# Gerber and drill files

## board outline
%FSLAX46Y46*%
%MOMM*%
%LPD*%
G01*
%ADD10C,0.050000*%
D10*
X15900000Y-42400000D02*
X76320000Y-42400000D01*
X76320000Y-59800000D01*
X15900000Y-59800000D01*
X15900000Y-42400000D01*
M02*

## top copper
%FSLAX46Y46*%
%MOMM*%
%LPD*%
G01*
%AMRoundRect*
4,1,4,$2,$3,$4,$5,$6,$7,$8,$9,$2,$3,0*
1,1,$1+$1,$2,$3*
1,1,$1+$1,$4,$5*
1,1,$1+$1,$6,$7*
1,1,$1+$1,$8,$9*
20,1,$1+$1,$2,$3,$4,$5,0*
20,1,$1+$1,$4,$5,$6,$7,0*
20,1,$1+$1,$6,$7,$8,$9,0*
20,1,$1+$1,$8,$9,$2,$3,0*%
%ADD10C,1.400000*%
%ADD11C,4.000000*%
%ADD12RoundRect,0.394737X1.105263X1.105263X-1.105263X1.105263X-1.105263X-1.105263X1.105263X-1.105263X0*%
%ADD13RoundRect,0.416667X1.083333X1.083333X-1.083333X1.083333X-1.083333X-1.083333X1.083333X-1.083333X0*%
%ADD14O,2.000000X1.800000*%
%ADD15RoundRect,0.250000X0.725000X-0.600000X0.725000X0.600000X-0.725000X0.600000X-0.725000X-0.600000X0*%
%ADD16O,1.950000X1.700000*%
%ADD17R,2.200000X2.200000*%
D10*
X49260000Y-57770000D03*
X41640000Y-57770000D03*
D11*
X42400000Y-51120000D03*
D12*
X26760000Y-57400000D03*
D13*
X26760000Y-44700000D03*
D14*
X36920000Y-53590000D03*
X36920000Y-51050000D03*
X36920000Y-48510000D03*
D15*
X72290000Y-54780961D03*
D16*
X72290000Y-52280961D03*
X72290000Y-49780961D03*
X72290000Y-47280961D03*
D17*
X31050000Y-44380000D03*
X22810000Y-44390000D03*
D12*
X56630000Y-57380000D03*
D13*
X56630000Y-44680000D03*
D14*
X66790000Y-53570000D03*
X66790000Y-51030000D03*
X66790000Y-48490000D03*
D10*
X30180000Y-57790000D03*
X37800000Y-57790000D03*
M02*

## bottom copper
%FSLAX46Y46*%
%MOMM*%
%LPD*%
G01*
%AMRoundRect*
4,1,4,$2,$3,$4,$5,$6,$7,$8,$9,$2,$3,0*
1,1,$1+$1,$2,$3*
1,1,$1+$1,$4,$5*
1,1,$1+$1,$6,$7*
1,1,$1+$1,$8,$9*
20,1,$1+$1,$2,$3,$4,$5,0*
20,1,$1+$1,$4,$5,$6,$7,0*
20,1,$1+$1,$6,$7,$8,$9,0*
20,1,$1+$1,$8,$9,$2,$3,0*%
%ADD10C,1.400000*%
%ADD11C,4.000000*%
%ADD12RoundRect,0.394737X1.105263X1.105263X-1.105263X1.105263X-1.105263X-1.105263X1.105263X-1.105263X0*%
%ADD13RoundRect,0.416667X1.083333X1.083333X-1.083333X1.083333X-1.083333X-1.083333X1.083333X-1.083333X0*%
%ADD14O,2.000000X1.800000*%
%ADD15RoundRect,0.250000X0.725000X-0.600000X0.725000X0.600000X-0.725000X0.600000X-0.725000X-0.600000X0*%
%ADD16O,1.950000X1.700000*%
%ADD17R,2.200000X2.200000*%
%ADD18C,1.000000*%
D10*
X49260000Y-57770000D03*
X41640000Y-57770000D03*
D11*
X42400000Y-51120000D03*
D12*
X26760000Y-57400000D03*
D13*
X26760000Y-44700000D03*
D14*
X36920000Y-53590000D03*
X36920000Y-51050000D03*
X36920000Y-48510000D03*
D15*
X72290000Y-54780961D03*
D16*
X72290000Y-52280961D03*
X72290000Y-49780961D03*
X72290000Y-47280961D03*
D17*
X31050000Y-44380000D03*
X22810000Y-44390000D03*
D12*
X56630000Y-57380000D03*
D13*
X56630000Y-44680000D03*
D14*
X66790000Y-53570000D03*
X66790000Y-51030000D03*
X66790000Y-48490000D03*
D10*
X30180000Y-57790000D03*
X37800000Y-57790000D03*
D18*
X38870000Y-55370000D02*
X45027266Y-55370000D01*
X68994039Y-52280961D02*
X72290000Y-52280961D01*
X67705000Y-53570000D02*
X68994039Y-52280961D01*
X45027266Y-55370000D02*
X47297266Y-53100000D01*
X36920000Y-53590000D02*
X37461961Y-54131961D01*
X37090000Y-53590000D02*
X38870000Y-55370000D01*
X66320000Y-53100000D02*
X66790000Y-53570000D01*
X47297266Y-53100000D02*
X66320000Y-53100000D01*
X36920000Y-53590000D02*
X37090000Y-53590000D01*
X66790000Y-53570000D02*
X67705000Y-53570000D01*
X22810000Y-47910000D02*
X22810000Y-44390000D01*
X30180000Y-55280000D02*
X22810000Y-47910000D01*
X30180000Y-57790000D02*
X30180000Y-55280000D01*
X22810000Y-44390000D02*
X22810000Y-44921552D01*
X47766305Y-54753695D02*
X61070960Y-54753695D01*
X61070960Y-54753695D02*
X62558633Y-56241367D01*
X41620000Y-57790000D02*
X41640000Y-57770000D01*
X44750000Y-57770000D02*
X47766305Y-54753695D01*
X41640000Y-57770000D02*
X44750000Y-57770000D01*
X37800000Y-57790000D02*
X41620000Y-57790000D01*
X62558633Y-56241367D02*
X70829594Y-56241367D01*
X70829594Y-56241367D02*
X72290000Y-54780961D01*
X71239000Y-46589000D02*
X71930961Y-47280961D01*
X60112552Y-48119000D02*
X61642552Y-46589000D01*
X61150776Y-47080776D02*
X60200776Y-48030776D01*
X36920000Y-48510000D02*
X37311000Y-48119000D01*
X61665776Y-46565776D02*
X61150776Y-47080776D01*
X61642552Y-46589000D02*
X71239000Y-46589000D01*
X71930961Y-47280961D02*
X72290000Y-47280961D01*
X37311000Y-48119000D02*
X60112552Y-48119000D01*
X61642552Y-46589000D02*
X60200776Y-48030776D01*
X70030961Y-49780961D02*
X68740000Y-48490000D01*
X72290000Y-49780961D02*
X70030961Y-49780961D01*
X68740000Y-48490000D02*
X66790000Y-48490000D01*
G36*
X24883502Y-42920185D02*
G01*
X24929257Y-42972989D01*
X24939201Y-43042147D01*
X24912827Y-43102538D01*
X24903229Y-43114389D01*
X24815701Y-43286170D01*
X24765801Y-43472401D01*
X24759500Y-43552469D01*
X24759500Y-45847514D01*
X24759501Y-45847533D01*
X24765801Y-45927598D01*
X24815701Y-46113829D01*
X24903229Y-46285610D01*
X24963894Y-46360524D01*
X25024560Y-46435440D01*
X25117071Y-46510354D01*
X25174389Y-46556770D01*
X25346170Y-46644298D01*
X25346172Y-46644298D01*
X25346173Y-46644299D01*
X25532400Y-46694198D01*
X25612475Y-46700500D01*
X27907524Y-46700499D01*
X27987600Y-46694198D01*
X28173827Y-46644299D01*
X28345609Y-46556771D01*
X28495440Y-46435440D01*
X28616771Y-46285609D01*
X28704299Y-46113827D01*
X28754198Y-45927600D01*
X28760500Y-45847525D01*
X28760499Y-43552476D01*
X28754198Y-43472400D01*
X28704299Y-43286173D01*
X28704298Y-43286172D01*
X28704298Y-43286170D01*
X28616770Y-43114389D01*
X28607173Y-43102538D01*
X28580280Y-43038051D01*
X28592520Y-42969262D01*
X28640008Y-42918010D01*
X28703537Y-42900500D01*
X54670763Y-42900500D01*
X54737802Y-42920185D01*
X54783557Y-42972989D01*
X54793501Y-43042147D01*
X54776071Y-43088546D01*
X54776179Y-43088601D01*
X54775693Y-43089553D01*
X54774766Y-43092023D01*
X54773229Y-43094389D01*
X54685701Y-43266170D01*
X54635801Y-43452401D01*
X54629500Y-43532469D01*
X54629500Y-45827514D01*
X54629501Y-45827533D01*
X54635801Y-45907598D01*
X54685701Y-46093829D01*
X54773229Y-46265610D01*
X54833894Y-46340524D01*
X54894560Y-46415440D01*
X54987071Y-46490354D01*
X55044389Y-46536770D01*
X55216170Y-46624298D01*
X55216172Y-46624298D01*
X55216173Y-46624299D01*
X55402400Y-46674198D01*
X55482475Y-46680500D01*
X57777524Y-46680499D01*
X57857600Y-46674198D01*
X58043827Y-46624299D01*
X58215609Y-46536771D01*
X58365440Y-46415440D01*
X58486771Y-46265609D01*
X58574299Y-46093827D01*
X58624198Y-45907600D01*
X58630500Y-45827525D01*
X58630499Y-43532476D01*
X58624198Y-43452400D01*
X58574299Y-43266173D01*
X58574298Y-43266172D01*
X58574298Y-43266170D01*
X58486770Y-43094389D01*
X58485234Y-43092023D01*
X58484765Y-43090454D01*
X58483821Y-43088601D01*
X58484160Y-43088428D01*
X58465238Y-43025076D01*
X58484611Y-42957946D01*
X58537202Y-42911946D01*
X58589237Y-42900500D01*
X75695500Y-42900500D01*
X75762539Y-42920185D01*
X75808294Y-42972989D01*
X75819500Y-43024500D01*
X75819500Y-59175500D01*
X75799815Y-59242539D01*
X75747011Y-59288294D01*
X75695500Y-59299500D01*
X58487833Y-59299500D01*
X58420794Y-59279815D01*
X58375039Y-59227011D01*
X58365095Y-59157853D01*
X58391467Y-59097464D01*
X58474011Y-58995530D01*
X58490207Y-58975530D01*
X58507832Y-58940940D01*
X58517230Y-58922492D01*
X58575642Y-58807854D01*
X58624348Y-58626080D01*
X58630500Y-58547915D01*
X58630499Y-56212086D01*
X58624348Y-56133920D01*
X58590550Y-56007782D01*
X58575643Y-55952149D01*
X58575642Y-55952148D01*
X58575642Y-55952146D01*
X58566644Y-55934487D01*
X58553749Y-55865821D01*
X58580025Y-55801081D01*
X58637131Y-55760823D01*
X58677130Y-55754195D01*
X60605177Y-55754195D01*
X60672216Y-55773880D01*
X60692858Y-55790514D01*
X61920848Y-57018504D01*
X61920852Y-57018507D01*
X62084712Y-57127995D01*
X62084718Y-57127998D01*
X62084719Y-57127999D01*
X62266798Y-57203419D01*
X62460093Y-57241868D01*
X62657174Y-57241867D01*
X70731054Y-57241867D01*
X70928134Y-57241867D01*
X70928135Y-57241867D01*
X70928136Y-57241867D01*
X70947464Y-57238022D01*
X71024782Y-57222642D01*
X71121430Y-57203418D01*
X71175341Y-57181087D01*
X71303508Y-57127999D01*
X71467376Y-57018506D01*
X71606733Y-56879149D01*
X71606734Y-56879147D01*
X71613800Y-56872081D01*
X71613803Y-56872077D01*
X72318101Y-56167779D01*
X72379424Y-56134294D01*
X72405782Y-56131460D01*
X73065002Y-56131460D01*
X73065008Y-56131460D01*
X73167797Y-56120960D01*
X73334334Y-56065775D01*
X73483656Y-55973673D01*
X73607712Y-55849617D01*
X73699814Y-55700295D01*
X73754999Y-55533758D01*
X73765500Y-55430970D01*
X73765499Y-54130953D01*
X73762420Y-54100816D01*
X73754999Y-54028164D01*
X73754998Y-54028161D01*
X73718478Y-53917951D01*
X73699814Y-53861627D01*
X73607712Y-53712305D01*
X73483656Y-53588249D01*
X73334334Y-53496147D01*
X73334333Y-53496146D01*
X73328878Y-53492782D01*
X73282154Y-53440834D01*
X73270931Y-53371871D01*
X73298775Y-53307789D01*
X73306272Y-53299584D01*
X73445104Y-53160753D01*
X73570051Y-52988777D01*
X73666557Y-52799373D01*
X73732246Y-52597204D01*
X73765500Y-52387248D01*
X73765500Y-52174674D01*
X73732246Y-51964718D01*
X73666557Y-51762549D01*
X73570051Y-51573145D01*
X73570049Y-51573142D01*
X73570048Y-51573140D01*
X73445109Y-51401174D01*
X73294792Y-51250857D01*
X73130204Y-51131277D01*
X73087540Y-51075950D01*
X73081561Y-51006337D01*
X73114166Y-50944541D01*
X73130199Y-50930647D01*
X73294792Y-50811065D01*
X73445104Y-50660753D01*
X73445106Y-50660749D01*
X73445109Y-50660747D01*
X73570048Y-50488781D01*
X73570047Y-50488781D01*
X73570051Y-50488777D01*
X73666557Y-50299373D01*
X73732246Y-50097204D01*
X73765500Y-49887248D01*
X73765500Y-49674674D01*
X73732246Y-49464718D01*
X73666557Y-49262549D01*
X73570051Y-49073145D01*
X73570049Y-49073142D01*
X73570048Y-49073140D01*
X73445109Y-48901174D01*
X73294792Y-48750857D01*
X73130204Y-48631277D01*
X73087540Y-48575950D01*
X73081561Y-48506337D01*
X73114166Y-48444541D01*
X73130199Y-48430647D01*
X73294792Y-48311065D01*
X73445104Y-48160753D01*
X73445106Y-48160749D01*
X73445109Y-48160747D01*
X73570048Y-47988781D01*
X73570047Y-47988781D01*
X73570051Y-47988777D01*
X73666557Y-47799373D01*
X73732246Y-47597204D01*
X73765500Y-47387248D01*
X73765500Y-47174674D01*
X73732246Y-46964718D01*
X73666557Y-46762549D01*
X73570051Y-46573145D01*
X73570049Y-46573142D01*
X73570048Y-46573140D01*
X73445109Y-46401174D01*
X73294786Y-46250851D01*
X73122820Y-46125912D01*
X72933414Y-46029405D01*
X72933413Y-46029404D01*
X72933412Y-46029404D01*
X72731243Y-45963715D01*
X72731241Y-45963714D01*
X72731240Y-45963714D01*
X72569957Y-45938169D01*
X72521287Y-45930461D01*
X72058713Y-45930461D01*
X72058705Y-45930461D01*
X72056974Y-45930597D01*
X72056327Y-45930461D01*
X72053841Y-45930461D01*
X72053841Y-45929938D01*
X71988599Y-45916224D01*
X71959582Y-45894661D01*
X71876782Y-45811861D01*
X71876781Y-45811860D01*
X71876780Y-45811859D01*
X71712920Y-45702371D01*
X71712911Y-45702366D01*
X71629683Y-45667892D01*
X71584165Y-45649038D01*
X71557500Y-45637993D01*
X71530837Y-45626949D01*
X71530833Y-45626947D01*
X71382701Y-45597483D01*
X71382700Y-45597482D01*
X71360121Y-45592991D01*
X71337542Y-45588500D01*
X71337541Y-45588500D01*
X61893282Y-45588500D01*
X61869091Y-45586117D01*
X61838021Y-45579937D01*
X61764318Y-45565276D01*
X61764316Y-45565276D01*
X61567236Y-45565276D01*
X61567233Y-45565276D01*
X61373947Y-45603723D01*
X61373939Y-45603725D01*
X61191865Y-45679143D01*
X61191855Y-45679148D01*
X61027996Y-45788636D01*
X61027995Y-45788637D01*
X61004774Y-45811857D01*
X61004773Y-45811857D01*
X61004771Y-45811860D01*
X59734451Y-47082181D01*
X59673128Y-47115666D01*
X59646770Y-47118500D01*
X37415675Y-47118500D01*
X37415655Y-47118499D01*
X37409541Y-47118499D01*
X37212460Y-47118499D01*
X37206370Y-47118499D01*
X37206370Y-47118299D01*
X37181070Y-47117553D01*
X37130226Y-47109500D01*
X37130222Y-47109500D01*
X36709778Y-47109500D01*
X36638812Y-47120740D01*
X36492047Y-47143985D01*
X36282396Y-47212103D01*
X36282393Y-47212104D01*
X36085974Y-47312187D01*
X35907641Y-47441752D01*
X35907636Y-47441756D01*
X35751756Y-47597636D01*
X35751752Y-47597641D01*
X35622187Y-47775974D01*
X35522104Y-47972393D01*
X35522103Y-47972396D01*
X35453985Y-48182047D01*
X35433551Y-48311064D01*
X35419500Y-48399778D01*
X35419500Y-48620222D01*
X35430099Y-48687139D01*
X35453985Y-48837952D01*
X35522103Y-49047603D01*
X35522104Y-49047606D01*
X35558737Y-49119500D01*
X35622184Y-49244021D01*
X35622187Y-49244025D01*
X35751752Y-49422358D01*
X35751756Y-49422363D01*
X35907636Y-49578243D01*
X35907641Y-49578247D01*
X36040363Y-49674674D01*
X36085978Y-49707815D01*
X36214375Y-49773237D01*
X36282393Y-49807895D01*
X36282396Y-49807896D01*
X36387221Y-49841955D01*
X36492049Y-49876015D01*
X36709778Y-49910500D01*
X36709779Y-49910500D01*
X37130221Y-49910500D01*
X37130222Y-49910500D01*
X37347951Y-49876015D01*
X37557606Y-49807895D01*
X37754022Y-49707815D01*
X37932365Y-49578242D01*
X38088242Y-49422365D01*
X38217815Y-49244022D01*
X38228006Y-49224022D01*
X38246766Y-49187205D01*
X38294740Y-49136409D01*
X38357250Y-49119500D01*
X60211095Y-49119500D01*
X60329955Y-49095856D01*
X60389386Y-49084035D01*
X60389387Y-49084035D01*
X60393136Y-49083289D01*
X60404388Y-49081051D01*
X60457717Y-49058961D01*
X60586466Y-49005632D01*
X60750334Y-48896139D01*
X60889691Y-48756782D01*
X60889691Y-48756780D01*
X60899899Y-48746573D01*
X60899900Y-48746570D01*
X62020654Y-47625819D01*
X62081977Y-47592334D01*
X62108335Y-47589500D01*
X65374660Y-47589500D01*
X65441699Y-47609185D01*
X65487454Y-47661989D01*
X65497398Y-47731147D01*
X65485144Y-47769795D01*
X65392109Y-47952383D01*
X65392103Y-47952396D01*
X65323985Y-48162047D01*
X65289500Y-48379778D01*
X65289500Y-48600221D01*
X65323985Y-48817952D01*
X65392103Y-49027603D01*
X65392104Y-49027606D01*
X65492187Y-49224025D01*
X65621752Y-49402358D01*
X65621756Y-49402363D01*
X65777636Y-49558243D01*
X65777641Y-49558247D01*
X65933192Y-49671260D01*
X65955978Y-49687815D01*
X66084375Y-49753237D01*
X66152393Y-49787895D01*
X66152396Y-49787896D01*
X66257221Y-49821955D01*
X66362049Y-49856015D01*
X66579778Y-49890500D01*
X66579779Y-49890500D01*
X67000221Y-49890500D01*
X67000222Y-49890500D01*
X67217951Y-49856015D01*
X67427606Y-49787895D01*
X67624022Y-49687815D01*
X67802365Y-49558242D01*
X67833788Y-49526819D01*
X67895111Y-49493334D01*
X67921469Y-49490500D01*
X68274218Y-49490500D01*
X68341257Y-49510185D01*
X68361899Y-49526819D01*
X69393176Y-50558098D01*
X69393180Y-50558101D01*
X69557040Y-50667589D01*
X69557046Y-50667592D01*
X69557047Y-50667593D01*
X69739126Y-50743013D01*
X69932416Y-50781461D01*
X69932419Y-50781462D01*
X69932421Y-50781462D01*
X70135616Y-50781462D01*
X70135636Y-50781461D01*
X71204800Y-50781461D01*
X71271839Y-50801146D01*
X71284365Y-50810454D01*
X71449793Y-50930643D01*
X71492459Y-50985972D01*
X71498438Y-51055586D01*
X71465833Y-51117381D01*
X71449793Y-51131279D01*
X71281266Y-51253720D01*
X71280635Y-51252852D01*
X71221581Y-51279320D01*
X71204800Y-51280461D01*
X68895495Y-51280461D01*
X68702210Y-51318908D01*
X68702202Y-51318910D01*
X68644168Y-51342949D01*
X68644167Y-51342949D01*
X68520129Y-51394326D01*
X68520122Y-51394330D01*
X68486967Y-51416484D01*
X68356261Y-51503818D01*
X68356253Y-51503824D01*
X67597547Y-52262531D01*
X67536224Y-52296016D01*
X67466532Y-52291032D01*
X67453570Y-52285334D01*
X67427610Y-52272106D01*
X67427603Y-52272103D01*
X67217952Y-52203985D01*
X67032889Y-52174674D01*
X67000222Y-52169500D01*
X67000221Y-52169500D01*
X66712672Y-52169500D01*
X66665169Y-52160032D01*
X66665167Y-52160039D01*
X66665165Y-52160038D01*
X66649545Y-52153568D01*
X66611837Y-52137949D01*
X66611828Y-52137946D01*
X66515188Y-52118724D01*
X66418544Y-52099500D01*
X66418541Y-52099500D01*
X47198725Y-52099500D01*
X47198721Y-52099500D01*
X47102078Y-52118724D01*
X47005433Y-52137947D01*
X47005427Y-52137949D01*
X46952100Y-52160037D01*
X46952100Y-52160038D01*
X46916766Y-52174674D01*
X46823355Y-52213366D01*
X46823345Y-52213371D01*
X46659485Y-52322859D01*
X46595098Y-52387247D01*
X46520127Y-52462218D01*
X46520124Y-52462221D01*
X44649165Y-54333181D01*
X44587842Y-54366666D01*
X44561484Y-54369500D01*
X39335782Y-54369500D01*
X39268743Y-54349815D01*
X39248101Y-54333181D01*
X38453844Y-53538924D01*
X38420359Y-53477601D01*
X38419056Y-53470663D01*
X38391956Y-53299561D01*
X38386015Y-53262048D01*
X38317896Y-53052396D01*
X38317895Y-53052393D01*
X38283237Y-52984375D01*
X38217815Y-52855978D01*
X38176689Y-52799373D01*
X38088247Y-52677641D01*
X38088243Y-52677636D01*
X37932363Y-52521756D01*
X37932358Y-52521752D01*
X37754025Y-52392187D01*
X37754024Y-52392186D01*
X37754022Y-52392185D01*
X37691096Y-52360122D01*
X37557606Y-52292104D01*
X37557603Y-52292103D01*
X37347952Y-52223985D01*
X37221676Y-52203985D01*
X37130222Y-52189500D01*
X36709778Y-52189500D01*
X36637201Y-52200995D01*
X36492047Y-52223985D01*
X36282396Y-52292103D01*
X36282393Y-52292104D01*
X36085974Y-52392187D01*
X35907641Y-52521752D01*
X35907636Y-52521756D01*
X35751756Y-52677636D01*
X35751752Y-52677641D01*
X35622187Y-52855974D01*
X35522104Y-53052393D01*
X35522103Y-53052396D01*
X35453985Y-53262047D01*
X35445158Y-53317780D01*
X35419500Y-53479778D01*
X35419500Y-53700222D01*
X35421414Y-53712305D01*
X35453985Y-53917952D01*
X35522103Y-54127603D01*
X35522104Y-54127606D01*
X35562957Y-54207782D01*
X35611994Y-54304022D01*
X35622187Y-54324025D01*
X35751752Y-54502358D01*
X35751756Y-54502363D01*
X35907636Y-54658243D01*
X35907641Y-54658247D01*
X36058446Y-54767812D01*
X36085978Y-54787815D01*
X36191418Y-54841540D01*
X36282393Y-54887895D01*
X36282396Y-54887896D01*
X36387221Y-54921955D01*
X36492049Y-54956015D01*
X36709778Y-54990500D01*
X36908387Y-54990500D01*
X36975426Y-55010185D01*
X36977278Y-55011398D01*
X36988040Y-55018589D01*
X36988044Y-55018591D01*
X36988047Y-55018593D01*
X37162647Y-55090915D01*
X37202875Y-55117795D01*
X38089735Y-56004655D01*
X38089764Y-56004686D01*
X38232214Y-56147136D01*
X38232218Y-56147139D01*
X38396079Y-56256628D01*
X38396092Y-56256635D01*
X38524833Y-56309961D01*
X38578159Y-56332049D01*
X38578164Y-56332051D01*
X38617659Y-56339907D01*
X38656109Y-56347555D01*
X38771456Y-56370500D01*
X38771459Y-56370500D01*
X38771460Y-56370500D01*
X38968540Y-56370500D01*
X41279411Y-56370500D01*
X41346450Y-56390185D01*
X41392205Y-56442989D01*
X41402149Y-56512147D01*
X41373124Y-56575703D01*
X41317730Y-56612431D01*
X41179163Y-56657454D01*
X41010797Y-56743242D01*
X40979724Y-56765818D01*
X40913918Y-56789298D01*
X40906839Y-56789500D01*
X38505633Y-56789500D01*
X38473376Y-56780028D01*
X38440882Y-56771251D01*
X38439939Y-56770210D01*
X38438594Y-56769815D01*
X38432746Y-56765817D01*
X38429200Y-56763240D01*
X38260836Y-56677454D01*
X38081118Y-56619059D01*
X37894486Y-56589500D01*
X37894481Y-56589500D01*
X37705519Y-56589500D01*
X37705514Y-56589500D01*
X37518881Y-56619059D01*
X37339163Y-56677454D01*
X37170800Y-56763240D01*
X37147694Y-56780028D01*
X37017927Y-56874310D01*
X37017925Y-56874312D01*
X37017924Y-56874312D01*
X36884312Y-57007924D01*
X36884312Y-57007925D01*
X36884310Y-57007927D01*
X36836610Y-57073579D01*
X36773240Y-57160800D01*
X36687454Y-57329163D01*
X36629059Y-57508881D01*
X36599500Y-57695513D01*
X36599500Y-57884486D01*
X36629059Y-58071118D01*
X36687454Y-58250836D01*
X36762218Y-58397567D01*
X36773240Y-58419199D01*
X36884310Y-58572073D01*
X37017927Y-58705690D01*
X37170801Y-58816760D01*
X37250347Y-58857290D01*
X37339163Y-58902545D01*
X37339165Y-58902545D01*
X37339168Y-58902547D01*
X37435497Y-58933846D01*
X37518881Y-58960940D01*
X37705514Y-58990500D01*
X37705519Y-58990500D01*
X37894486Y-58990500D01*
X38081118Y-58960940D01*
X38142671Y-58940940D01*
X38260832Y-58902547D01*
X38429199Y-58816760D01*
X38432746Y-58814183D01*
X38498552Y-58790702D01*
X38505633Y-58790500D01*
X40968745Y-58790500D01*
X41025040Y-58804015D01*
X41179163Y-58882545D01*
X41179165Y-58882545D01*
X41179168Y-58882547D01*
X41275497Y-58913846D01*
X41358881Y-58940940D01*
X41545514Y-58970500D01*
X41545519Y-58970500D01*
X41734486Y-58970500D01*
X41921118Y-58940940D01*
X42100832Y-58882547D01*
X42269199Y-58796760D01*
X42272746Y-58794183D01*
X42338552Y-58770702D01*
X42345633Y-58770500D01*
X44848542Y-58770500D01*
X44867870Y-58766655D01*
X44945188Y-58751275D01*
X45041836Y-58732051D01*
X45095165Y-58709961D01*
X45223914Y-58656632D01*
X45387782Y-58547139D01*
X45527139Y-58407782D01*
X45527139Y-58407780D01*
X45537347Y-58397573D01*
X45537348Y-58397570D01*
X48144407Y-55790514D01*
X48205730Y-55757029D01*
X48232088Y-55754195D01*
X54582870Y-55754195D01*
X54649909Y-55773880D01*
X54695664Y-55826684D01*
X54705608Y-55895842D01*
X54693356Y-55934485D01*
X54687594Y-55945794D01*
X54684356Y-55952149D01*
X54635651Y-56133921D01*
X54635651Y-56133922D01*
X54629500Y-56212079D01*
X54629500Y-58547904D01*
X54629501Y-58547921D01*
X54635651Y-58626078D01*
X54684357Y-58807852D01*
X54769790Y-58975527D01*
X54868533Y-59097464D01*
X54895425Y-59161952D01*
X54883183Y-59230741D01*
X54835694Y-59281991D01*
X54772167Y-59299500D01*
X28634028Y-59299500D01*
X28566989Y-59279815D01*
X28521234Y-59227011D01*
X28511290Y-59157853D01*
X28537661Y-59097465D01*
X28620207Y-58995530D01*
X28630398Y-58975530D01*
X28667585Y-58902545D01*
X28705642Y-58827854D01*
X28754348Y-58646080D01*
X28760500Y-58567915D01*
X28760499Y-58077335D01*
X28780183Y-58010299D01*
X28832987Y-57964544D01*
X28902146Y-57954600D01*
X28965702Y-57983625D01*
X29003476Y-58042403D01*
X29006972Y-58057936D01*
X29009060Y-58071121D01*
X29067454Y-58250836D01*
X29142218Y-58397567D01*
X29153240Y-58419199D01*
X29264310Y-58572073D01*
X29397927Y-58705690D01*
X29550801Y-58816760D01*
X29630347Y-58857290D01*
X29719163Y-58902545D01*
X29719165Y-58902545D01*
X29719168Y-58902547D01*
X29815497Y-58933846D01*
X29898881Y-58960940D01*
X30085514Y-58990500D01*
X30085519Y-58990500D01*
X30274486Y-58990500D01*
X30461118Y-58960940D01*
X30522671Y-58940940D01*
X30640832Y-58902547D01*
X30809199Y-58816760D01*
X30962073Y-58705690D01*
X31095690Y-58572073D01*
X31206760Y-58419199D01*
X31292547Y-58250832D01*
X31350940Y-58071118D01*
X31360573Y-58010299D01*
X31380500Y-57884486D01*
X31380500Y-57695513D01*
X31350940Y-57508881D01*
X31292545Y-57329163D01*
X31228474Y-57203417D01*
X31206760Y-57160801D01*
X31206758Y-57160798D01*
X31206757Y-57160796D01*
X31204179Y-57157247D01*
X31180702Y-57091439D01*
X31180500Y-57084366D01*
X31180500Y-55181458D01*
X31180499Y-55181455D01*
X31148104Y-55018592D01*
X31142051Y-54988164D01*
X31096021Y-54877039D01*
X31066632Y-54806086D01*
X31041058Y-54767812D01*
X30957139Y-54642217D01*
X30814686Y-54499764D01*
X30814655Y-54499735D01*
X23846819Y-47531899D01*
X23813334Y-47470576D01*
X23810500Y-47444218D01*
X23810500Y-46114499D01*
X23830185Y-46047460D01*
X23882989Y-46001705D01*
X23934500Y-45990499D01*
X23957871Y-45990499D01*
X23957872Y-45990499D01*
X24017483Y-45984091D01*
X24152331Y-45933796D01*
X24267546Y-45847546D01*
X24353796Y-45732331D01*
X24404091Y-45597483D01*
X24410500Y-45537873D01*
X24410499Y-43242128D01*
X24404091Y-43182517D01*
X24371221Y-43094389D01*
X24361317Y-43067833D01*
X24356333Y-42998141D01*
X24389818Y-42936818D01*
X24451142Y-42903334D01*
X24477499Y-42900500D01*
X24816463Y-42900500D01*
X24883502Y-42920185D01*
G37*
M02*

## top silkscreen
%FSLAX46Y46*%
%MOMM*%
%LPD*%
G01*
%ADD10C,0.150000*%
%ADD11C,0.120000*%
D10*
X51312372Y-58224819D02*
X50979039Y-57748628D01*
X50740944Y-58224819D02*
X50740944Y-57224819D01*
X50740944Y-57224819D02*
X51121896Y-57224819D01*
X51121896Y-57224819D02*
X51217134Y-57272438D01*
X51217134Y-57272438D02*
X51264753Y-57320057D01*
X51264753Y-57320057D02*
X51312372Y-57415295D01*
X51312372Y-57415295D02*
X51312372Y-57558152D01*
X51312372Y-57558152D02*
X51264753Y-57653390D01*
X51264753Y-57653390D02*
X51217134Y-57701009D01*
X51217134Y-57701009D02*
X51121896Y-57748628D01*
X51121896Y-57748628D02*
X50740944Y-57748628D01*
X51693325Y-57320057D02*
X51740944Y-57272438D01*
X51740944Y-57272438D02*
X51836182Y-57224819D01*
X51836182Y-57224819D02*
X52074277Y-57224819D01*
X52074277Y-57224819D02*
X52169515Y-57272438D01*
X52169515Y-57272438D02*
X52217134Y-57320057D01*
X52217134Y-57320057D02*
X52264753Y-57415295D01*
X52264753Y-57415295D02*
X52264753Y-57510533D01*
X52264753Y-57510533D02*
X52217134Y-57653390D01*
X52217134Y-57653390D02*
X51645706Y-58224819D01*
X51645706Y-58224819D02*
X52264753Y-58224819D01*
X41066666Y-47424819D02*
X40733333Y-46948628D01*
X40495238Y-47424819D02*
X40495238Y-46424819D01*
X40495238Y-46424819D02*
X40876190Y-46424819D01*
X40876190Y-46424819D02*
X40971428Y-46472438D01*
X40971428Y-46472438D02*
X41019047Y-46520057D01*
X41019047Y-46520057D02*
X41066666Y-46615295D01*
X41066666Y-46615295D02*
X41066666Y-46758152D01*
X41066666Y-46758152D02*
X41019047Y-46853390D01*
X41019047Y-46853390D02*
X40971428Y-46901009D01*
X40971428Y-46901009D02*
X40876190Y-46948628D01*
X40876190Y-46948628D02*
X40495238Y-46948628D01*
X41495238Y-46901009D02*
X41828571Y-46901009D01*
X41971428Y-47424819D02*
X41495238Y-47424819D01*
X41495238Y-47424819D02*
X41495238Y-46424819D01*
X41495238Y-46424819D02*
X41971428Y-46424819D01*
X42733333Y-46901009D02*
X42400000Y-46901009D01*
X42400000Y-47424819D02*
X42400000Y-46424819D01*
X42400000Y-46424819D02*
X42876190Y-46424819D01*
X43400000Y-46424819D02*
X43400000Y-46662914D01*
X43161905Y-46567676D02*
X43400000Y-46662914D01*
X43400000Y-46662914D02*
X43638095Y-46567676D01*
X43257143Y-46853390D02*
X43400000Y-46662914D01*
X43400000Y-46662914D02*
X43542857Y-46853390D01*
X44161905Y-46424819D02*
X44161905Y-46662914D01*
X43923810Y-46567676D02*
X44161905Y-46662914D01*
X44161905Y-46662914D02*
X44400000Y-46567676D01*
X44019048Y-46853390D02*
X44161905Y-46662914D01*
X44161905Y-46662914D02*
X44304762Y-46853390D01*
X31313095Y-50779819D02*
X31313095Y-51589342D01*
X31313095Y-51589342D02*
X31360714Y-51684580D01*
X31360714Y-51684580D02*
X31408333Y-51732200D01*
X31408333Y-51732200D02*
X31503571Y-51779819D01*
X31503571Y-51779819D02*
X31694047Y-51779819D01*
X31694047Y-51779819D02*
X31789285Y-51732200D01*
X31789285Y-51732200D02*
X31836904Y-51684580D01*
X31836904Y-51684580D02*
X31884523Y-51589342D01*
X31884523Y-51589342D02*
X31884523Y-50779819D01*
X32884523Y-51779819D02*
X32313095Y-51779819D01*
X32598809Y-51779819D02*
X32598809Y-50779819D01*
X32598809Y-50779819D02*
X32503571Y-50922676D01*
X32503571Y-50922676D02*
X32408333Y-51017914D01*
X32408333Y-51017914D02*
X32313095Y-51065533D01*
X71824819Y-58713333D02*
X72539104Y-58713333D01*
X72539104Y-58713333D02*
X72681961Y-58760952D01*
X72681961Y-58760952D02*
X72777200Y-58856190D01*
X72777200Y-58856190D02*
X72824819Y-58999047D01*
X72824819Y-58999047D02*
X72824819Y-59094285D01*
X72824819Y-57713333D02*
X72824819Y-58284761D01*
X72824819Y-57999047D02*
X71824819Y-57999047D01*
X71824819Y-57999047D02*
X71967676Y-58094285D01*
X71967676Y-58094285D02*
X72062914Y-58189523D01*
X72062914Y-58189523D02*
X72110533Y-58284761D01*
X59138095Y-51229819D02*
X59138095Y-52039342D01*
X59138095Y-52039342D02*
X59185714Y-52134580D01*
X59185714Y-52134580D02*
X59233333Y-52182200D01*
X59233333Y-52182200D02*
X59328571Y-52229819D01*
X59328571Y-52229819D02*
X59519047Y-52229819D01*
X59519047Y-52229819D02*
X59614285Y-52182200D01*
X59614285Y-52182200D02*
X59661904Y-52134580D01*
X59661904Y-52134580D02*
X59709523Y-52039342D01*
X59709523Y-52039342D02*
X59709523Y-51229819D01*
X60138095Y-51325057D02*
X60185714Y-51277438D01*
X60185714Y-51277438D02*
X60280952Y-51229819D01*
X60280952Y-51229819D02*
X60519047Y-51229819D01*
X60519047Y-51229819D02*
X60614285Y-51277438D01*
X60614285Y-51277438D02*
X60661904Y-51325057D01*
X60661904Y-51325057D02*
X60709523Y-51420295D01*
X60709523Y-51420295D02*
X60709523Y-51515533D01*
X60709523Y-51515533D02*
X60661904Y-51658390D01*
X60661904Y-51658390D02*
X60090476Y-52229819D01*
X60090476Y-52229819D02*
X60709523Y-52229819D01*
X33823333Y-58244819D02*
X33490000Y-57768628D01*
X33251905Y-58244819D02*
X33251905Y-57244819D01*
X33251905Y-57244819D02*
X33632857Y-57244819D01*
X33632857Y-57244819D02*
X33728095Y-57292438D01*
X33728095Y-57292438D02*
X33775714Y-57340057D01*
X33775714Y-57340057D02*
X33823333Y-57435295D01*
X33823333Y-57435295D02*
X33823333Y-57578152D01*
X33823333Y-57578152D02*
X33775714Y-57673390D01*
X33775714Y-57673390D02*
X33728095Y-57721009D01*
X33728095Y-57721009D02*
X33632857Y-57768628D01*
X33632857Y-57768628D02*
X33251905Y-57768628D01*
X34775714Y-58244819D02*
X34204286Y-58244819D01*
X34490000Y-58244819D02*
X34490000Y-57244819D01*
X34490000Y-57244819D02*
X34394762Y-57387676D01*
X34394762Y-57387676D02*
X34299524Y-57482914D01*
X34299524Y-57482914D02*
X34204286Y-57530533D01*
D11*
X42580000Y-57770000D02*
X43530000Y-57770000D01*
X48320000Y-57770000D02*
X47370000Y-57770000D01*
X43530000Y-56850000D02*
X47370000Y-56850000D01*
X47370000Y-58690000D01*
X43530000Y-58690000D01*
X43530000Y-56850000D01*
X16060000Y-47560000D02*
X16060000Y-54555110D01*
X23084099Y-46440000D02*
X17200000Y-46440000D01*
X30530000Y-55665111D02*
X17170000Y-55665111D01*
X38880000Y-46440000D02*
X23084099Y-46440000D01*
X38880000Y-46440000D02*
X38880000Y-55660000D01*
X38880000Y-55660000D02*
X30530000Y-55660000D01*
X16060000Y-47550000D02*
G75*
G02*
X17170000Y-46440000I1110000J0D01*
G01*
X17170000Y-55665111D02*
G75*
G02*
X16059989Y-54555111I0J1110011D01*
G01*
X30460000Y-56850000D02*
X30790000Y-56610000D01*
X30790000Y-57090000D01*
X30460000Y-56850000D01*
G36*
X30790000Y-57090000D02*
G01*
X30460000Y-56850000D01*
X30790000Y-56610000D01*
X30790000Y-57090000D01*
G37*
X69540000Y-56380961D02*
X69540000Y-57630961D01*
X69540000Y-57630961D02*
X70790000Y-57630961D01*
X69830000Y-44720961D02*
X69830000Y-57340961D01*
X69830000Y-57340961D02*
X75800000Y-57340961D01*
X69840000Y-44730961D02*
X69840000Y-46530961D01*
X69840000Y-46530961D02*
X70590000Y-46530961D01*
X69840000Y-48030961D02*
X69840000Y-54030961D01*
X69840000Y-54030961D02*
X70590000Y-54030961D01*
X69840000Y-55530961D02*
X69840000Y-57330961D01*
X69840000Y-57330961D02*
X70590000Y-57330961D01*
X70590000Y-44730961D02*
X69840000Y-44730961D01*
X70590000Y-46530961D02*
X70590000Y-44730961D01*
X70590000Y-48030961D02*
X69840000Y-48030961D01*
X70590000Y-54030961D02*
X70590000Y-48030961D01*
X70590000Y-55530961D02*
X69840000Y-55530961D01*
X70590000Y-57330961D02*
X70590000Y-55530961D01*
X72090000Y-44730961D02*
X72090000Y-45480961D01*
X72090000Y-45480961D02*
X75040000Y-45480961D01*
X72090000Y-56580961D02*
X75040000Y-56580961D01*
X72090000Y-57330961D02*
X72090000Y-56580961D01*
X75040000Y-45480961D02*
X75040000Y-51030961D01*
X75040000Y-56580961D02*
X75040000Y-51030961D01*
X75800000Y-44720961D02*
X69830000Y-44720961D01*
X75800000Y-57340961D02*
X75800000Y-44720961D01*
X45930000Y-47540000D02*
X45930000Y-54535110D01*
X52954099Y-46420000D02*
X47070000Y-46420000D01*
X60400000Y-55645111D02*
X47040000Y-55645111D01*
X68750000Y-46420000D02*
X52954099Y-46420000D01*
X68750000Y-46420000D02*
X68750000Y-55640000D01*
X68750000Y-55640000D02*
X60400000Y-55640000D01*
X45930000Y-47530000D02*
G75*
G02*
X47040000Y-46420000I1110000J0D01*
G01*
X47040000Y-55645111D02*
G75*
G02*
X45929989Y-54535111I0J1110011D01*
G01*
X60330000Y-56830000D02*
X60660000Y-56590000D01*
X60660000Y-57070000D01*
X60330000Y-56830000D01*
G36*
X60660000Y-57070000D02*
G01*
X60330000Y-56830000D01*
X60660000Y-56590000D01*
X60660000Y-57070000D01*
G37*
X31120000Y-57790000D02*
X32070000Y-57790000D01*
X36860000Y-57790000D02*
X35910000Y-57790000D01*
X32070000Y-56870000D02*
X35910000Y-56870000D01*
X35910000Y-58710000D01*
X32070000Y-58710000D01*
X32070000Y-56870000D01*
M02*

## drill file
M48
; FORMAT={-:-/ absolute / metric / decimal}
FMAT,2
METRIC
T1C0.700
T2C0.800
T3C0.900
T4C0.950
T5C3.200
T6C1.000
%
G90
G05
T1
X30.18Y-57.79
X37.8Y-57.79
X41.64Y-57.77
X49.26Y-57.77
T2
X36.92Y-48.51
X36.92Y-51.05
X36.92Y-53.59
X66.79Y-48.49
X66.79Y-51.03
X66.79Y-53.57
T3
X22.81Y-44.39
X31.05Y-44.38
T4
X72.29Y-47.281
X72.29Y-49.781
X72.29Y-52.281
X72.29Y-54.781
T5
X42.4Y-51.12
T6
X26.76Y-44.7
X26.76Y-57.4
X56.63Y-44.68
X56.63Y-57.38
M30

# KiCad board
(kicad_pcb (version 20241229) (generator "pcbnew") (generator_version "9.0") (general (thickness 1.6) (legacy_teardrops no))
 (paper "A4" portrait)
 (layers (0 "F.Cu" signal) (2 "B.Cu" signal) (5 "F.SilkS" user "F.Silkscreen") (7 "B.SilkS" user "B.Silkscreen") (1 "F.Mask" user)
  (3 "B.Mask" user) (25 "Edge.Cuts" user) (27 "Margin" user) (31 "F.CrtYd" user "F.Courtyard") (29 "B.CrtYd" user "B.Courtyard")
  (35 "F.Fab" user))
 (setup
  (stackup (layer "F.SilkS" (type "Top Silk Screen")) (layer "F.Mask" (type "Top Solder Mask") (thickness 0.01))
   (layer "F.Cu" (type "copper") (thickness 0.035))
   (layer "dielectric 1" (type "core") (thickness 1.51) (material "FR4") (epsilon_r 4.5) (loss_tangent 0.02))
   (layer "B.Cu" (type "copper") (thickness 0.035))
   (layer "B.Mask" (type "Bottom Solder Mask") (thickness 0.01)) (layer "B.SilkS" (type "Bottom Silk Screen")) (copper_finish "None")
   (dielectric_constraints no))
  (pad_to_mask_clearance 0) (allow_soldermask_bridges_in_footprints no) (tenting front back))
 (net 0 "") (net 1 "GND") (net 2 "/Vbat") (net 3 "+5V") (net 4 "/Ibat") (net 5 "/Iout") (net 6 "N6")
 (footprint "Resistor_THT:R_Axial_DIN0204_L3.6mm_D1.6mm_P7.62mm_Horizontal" (layer "F.Cu") (at 49.26 57.77 180)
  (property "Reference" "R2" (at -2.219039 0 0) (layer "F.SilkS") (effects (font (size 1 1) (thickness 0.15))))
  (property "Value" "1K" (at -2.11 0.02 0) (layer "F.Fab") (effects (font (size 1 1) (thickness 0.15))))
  (fp_line (start 6.68 0) (end 5.73 0) (stroke (width 0.12) (type solid)) (layer "F.SilkS"))
  (fp_line (start 0.94 0) (end 1.89 0) (stroke (width 0.12) (type solid)) (layer "F.SilkS"))
  (fp_rect (start 1.89 -0.92) (end 5.73 0.92) (stroke (width 0.12) (type solid)) (fill no) (layer "F.SilkS"))
  (pad "1" thru_hole circle (at 0 0 180) (size 1.4 1.4) (drill 0.7) (layers "*.Cu" "*.Mask") (remove_unused_layers no) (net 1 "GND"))
  (pad "2" thru_hole circle (at 7.62 0 180) (size 1.4 1.4) (drill 0.7) (layers "*.Cu" "*.Mask") (remove_unused_layers no) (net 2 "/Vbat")))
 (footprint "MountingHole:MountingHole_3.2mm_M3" (layer "F.Cu") (at 42.4 51.12)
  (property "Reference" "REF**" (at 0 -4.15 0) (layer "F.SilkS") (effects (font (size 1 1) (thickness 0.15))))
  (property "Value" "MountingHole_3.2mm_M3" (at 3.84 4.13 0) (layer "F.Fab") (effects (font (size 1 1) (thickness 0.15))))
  (pad "" thru_hole circle (at 0 0) (size 4 4) (drill 3.2) (layers "*.Cu" "*.Mask") (remove_unused_layers no) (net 1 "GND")))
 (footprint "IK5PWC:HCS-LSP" (layer "F.Cu") (at 29.26 56.85 180)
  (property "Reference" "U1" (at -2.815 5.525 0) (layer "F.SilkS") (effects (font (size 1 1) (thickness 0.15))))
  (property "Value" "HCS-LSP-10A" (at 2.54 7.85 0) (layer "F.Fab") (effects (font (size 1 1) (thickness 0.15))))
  (fp_line (start 13.2 9.29) (end 13.2 2.29489) (stroke (width 0.12) (type solid)) (layer "F.SilkS"))
  (fp_line (start 6.175901 10.41) (end 12.06 10.41) (stroke (width 0.12) (type solid)) (layer "F.SilkS"))
  (fp_line (start -1.27 1.184889) (end 12.09 1.184889) (stroke (width 0.12) (type solid)) (layer "F.SilkS"))
  (fp_line (start -9.62 10.41) (end 6.175901 10.41) (stroke (width 0.12) (type solid)) (layer "F.SilkS"))
  (fp_line (start -9.62 10.41) (end -9.62 1.19) (stroke (width 0.12) (type solid)) (layer "F.SilkS"))
  (fp_line (start -9.62 1.19) (end -1.27 1.19) (stroke (width 0.12) (type solid)) (layer "F.SilkS"))
  (fp_arc (start 13.2 9.3) (mid 12.874889 10.084889) (end 12.09 10.41) (stroke (width 0.12) (type solid)) (layer "F.SilkS"))
  (fp_arc (start 12.09 1.184889) (mid 12.874889 1.51) (end 13.2 2.294889) (stroke (width 0.12) (type solid)) (layer "F.SilkS"))
  (fp_poly (pts (xy -1.2 0) (xy -1.53 0.24) (xy -1.53 -0.24) (xy -1.2 0)) (stroke (width 0.12) (type solid)) (fill yes) (layer "F.SilkS"))
  (pad "" np_thru_hole roundrect (at 2.5 -0.55 180) (size 3 3) (drill 1) (layers "*.Cu" "*.Mask") (roundrect_rratio 0.1315789474))
  (pad "" np_thru_hole roundrect (at 2.5 12.15 180) (size 3 3) (drill 1) (layers "*.Cu" "*.Mask") (roundrect_rratio 0.1388888889))
  (pad "1" thru_hole oval (at -7.66 3.26 180) (size 2 1.8) (drill 0.8) (layers "*.Cu" "*.Mask") (remove_unused_layers no) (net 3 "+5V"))
  (pad "2" thru_hole oval (at -7.66 5.8 180) (size 2 1.8) (drill 0.8) (layers "*.Cu" "*.Mask") (remove_unused_layers no) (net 1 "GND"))
  (pad "3" thru_hole oval (at -7.66 8.34 180) (size 2 1.8) (drill 0.8) (layers "*.Cu" "*.Mask") (remove_unused_layers no) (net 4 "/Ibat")))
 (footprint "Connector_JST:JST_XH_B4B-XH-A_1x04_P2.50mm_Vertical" (layer "F.Cu") (at 72.29 54.780961 90)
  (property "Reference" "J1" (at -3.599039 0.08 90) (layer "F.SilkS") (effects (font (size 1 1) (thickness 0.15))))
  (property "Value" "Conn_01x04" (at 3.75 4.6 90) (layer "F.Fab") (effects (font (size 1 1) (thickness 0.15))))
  (fp_line (start -1.6 -2.75) (end -2.85 -2.75) (stroke (width 0.12) (type solid)) (layer "F.SilkS"))
  (fp_line (start -2.85 -2.75) (end -2.85 -1.5) (stroke (width 0.12) (type solid)) (layer "F.SilkS"))
  (fp_line (start 10.06 -2.46) (end -2.56 -2.46) (stroke (width 0.12) (type solid)) (layer "F.SilkS"))
  (fp_line (start -2.56 -2.46) (end -2.56 3.51) (stroke (width 0.12) (type solid)) (layer "F.SilkS"))
  (fp_line (start 10.05 -2.45) (end 8.25 -2.45) (stroke (width 0.12) (type solid)) (layer "F.SilkS"))
  (fp_line (start 8.25 -2.45) (end 8.25 -1.7) (stroke (width 0.12) (type solid)) (layer "F.SilkS"))
  (fp_line (start 6.75 -2.45) (end 0.75 -2.45) (stroke (width 0.12) (type solid)) (layer "F.SilkS"))
  (fp_line (start 0.75 -2.45) (end 0.75 -1.7) (stroke (width 0.12) (type solid)) (layer "F.SilkS"))
  (fp_line (start -0.75 -2.45) (end -2.55 -2.45) (stroke (width 0.12) (type solid)) (layer "F.SilkS"))
  (fp_line (start -2.55 -2.45) (end -2.55 -1.7) (stroke (width 0.12) (type solid)) (layer "F.SilkS"))
  (fp_line (start 10.05 -1.7) (end 10.05 -2.45) (stroke (width 0.12) (type solid)) (layer "F.SilkS"))
  (fp_line (start 8.25 -1.7) (end 10.05 -1.7) (stroke (width 0.12) (type solid)) (layer "F.SilkS"))
  (fp_line (start 6.75 -1.7) (end 6.75 -2.45) (stroke (width 0.12) (type solid)) (layer "F.SilkS"))
  (fp_line (start 0.75 -1.7) (end 6.75 -1.7) (stroke (width 0.12) (type solid)) (layer "F.SilkS"))
  (fp_line (start -0.75 -1.7) (end -0.75 -2.45) (stroke (width 0.12) (type solid)) (layer "F.SilkS"))
  (fp_line (start -2.55 -1.7) (end -0.75 -1.7) (stroke (width 0.12) (type solid)) (layer "F.SilkS"))
  (fp_line (start 10.05 -0.2) (end 9.3 -0.2) (stroke (width 0.12) (type solid)) (layer "F.SilkS"))
  (fp_line (start 9.3 -0.2) (end 9.3 2.75) (stroke (width 0.12) (type solid)) (layer "F.SilkS"))
  (fp_line (start -1.8 -0.2) (end -1.8 2.75) (stroke (width 0.12) (type solid)) (layer "F.SilkS"))
  (fp_line (start -2.55 -0.2) (end -1.8 -0.2) (stroke (width 0.12) (type solid)) (layer "F.SilkS"))
  (fp_line (start 9.3 2.75) (end 3.75 2.75) (stroke (width 0.12) (type solid)) (layer "F.SilkS"))
  (fp_line (start -1.8 2.75) (end 3.75 2.75) (stroke (width 0.12) (type solid)) (layer "F.SilkS"))
  (fp_line (start 10.06 3.51) (end 10.06 -2.46) (stroke (width 0.12) (type solid)) (layer "F.SilkS"))
  (fp_line (start -2.56 3.51) (end 10.06 3.51) (stroke (width 0.12) (type solid)) (layer "F.SilkS"))
  (pad "1" thru_hole roundrect (at 0 0 90) (size 1.7 1.95) (drill 0.95) (layers "*.Cu" "*.Mask") (remove_unused_layers no)
   (roundrect_rratio 0.147059) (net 2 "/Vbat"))
  (pad "2" thru_hole oval (at 2.5 0 90) (size 1.7 1.95) (drill 0.95) (layers "*.Cu" "*.Mask") (remove_unused_layers no) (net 3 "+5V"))
  (pad "3" thru_hole oval (at 5 0 90) (size 1.7 1.95) (drill 0.95) (layers "*.Cu" "*.Mask") (remove_unused_layers no) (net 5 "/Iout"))
  (pad "4" thru_hole oval (at 7.5 0 90) (size 1.7 1.95) (drill 0.95) (layers "*.Cu" "*.Mask") (remove_unused_layers no) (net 4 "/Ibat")))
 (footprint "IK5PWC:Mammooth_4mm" (layer "F.Cu") (at 31.05 44.38 180)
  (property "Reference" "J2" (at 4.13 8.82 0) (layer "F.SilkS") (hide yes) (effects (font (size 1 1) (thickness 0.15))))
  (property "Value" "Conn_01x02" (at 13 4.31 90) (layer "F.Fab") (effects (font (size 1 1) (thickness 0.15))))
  (pad "1" thru_hole rect (at 0 0 180) (size 2.2 2.2) (drill 0.9) (layers "*.Cu" "*.Mask") (remove_unused_layers no) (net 1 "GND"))
  (pad "2" thru_hole rect (at 8.24 -0.01 180) (size 2.2 2.2) (drill 0.9) (layers "*.Cu" "*.Mask") (remove_unused_layers no) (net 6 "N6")))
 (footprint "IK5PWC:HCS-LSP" (layer "F.Cu") (at 59.13 56.83 180)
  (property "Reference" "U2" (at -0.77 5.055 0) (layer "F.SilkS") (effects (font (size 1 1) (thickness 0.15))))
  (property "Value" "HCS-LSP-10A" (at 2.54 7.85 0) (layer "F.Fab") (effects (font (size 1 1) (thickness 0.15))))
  (fp_line (start 13.2 9.29) (end 13.2 2.29489) (stroke (width 0.12) (type solid)) (layer "F.SilkS"))
  (fp_line (start 6.175901 10.41) (end 12.06 10.41) (stroke (width 0.12) (type solid)) (layer "F.SilkS"))
  (fp_line (start -1.27 1.184889) (end 12.09 1.184889) (stroke (width 0.12) (type solid)) (layer "F.SilkS"))
  (fp_line (start -9.62 10.41) (end 6.175901 10.41) (stroke (width 0.12) (type solid)) (layer "F.SilkS"))
  (fp_line (start -9.62 10.41) (end -9.62 1.19) (stroke (width 0.12) (type solid)) (layer "F.SilkS"))
  (fp_line (start -9.62 1.19) (end -1.27 1.19) (stroke (width 0.12) (type solid)) (layer "F.SilkS"))
  (fp_arc (start 13.2 9.3) (mid 12.874889 10.084889) (end 12.09 10.41) (stroke (width 0.12) (type solid)) (layer "F.SilkS"))
  (fp_arc (start 12.09 1.184889) (mid 12.874889 1.51) (end 13.2 2.294889) (stroke (width 0.12) (type solid)) (layer "F.SilkS"))
  (fp_poly (pts (xy -1.2 0) (xy -1.53 0.24) (xy -1.53 -0.24) (xy -1.2 0)) (stroke (width 0.12) (type solid)) (fill yes) (layer "F.SilkS"))
  (pad "" np_thru_hole roundrect (at 2.5 -0.55 180) (size 3 3) (drill 1) (layers "*.Cu" "*.Mask") (roundrect_rratio 0.1315789474))
  (pad "" np_thru_hole roundrect (at 2.5 12.15 180) (size 3 3) (drill 1) (layers "*.Cu" "*.Mask") (roundrect_rratio 0.1388888889))
  (pad "1" thru_hole oval (at -7.66 3.26 180) (size 2 1.8) (drill 0.8) (layers "*.Cu" "*.Mask") (remove_unused_layers no) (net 3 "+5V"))
  (pad "2" thru_hole oval (at -7.66 5.8 180) (size 2 1.8) (drill 0.8) (layers "*.Cu" "*.Mask") (remove_unused_layers no) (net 1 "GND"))
  (pad "3" thru_hole oval (at -7.66 8.34 180) (size 2 1.8) (drill 0.8) (layers "*.Cu" "*.Mask") (remove_unused_layers no) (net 5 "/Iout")))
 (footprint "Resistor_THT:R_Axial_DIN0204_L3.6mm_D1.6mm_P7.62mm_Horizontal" (layer "F.Cu") (at 30.18 57.79)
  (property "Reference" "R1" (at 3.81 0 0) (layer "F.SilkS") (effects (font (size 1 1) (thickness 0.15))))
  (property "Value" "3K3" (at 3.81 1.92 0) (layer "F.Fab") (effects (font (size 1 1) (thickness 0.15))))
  (fp_line (start 0.94 0) (end 1.89 0) (stroke (width 0.12) (type solid)) (layer "F.SilkS"))
  (fp_line (start 6.68 0) (end 5.73 0) (stroke (width 0.12) (type solid)) (layer "F.SilkS"))
  (fp_rect (start 1.89 -0.92) (end 5.73 0.92) (stroke (width 0.12) (type solid)) (fill no) (layer "F.SilkS"))
  (pad "1" thru_hole circle (at 0 0) (size 1.4 1.4) (drill 0.7) (layers "*.Cu" "*.Mask") (remove_unused_layers no) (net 6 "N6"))
  (pad "2" thru_hole circle (at 7.62 0) (size 1.4 1.4) (drill 0.7) (layers "*.Cu" "*.Mask") (remove_unused_layers no) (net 2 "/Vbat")))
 (gr_rect (start 15.9 42.4) (end 76.32 59.8) (stroke (width 0.05) (type solid)) (fill no) (layer "Edge.Cuts"))
 (segment (start 38.87 55.37) (end 45.027266 55.37) (width 1) (layer "B.Cu") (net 3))
 (segment (start 68.994039 52.280961) (end 72.29 52.280961) (width 1) (layer "B.Cu") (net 3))
 (segment (start 67.705 53.57) (end 68.994039 52.280961) (width 1) (layer "B.Cu") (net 3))
 (segment (start 45.027266 55.37) (end 47.297266 53.1) (width 1) (layer "B.Cu") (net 3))
 (segment (start 36.92 53.59) (end 37.461961 54.131961) (width 1) (layer "B.Cu") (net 3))
 (segment (start 37.09 53.59) (end 38.87 55.37) (width 1) (layer "B.Cu") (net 3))
 (segment (start 66.32 53.1) (end 66.79 53.57) (width 1) (layer "B.Cu") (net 3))
 (segment (start 47.297266 53.1) (end 66.32 53.1) (width 1) (layer "B.Cu") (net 3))
 (segment (start 36.92 53.59) (end 37.09 53.59) (width 1) (layer "B.Cu") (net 3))
 (segment (start 66.79 53.57) (end 67.705 53.57) (width 1) (layer "B.Cu") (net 3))
 (segment (start 22.81 47.91) (end 22.81 44.39) (width 1) (layer "B.Cu") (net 6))
 (segment (start 30.18 55.28) (end 22.81 47.91) (width 1) (layer "B.Cu") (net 6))
 (segment (start 30.18 57.79) (end 30.18 55.28) (width 1) (layer "B.Cu") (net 6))
 (segment (start 22.81 44.39) (end 22.81 44.921552) (width 1) (layer "B.Cu") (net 6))
 (segment (start 47.766305 54.753695) (end 61.07096 54.753695) (width 1) (layer "B.Cu") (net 2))
 (segment (start 61.07096 54.753695) (end 62.558633 56.241367) (width 1) (layer "B.Cu") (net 2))
 (segment (start 41.62 57.79) (end 41.64 57.77) (width 1) (layer "B.Cu") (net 2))
 (segment (start 44.75 57.77) (end 47.766305 54.753695) (width 1) (layer "B.Cu") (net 2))
 (segment (start 41.64 57.77) (end 44.75 57.77) (width 1) (layer "B.Cu") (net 2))
 (segment (start 37.8 57.79) (end 41.62 57.79) (width 1) (layer "B.Cu") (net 2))
 (segment (start 62.558633 56.241367) (end 70.829594 56.241367) (width 1) (layer "B.Cu") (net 2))
 (segment (start 70.829594 56.241367) (end 72.29 54.780961) (width 1) (layer "B.Cu") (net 2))
 (segment (start 71.239 46.589) (end 71.930961 47.280961) (width 1) (layer "B.Cu") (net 4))
 (segment (start 60.112552 48.119) (end 61.642552 46.589) (width 1) (layer "B.Cu") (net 4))
 (segment (start 61.150776 47.080776) (end 60.200776 48.030776) (width 1) (layer "B.Cu") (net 4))
 (segment (start 36.92 48.51) (end 37.311 48.119) (width 1) (layer "B.Cu") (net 4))
 (segment (start 61.665776 46.565776) (end 61.150776 47.080776) (width 1) (layer "B.Cu") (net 4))
 (segment (start 61.642552 46.589) (end 71.239 46.589) (width 1) (layer "B.Cu") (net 4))
 (segment (start 71.930961 47.280961) (end 72.29 47.280961) (width 1) (layer "B.Cu") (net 4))
 (segment (start 37.311 48.119) (end 60.112552 48.119) (width 1) (layer "B.Cu") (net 4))
 (segment (start 61.642552 46.589) (end 60.200776 48.030776) (width 1) (layer "B.Cu") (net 4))
 (segment (start 70.030961 49.780961) (end 68.74 48.49) (width 1) (layer "B.Cu") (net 5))
 (segment (start 72.29 49.780961) (end 70.030961 49.780961) (width 1) (layer "B.Cu") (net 5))
 (segment (start 68.74 48.49) (end 66.79 48.49) (width 1) (layer "B.Cu") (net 5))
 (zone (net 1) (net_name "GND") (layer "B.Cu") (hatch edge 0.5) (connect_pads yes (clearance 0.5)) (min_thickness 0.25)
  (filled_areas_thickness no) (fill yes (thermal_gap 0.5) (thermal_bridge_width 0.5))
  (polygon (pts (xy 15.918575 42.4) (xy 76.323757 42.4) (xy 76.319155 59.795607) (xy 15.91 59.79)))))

